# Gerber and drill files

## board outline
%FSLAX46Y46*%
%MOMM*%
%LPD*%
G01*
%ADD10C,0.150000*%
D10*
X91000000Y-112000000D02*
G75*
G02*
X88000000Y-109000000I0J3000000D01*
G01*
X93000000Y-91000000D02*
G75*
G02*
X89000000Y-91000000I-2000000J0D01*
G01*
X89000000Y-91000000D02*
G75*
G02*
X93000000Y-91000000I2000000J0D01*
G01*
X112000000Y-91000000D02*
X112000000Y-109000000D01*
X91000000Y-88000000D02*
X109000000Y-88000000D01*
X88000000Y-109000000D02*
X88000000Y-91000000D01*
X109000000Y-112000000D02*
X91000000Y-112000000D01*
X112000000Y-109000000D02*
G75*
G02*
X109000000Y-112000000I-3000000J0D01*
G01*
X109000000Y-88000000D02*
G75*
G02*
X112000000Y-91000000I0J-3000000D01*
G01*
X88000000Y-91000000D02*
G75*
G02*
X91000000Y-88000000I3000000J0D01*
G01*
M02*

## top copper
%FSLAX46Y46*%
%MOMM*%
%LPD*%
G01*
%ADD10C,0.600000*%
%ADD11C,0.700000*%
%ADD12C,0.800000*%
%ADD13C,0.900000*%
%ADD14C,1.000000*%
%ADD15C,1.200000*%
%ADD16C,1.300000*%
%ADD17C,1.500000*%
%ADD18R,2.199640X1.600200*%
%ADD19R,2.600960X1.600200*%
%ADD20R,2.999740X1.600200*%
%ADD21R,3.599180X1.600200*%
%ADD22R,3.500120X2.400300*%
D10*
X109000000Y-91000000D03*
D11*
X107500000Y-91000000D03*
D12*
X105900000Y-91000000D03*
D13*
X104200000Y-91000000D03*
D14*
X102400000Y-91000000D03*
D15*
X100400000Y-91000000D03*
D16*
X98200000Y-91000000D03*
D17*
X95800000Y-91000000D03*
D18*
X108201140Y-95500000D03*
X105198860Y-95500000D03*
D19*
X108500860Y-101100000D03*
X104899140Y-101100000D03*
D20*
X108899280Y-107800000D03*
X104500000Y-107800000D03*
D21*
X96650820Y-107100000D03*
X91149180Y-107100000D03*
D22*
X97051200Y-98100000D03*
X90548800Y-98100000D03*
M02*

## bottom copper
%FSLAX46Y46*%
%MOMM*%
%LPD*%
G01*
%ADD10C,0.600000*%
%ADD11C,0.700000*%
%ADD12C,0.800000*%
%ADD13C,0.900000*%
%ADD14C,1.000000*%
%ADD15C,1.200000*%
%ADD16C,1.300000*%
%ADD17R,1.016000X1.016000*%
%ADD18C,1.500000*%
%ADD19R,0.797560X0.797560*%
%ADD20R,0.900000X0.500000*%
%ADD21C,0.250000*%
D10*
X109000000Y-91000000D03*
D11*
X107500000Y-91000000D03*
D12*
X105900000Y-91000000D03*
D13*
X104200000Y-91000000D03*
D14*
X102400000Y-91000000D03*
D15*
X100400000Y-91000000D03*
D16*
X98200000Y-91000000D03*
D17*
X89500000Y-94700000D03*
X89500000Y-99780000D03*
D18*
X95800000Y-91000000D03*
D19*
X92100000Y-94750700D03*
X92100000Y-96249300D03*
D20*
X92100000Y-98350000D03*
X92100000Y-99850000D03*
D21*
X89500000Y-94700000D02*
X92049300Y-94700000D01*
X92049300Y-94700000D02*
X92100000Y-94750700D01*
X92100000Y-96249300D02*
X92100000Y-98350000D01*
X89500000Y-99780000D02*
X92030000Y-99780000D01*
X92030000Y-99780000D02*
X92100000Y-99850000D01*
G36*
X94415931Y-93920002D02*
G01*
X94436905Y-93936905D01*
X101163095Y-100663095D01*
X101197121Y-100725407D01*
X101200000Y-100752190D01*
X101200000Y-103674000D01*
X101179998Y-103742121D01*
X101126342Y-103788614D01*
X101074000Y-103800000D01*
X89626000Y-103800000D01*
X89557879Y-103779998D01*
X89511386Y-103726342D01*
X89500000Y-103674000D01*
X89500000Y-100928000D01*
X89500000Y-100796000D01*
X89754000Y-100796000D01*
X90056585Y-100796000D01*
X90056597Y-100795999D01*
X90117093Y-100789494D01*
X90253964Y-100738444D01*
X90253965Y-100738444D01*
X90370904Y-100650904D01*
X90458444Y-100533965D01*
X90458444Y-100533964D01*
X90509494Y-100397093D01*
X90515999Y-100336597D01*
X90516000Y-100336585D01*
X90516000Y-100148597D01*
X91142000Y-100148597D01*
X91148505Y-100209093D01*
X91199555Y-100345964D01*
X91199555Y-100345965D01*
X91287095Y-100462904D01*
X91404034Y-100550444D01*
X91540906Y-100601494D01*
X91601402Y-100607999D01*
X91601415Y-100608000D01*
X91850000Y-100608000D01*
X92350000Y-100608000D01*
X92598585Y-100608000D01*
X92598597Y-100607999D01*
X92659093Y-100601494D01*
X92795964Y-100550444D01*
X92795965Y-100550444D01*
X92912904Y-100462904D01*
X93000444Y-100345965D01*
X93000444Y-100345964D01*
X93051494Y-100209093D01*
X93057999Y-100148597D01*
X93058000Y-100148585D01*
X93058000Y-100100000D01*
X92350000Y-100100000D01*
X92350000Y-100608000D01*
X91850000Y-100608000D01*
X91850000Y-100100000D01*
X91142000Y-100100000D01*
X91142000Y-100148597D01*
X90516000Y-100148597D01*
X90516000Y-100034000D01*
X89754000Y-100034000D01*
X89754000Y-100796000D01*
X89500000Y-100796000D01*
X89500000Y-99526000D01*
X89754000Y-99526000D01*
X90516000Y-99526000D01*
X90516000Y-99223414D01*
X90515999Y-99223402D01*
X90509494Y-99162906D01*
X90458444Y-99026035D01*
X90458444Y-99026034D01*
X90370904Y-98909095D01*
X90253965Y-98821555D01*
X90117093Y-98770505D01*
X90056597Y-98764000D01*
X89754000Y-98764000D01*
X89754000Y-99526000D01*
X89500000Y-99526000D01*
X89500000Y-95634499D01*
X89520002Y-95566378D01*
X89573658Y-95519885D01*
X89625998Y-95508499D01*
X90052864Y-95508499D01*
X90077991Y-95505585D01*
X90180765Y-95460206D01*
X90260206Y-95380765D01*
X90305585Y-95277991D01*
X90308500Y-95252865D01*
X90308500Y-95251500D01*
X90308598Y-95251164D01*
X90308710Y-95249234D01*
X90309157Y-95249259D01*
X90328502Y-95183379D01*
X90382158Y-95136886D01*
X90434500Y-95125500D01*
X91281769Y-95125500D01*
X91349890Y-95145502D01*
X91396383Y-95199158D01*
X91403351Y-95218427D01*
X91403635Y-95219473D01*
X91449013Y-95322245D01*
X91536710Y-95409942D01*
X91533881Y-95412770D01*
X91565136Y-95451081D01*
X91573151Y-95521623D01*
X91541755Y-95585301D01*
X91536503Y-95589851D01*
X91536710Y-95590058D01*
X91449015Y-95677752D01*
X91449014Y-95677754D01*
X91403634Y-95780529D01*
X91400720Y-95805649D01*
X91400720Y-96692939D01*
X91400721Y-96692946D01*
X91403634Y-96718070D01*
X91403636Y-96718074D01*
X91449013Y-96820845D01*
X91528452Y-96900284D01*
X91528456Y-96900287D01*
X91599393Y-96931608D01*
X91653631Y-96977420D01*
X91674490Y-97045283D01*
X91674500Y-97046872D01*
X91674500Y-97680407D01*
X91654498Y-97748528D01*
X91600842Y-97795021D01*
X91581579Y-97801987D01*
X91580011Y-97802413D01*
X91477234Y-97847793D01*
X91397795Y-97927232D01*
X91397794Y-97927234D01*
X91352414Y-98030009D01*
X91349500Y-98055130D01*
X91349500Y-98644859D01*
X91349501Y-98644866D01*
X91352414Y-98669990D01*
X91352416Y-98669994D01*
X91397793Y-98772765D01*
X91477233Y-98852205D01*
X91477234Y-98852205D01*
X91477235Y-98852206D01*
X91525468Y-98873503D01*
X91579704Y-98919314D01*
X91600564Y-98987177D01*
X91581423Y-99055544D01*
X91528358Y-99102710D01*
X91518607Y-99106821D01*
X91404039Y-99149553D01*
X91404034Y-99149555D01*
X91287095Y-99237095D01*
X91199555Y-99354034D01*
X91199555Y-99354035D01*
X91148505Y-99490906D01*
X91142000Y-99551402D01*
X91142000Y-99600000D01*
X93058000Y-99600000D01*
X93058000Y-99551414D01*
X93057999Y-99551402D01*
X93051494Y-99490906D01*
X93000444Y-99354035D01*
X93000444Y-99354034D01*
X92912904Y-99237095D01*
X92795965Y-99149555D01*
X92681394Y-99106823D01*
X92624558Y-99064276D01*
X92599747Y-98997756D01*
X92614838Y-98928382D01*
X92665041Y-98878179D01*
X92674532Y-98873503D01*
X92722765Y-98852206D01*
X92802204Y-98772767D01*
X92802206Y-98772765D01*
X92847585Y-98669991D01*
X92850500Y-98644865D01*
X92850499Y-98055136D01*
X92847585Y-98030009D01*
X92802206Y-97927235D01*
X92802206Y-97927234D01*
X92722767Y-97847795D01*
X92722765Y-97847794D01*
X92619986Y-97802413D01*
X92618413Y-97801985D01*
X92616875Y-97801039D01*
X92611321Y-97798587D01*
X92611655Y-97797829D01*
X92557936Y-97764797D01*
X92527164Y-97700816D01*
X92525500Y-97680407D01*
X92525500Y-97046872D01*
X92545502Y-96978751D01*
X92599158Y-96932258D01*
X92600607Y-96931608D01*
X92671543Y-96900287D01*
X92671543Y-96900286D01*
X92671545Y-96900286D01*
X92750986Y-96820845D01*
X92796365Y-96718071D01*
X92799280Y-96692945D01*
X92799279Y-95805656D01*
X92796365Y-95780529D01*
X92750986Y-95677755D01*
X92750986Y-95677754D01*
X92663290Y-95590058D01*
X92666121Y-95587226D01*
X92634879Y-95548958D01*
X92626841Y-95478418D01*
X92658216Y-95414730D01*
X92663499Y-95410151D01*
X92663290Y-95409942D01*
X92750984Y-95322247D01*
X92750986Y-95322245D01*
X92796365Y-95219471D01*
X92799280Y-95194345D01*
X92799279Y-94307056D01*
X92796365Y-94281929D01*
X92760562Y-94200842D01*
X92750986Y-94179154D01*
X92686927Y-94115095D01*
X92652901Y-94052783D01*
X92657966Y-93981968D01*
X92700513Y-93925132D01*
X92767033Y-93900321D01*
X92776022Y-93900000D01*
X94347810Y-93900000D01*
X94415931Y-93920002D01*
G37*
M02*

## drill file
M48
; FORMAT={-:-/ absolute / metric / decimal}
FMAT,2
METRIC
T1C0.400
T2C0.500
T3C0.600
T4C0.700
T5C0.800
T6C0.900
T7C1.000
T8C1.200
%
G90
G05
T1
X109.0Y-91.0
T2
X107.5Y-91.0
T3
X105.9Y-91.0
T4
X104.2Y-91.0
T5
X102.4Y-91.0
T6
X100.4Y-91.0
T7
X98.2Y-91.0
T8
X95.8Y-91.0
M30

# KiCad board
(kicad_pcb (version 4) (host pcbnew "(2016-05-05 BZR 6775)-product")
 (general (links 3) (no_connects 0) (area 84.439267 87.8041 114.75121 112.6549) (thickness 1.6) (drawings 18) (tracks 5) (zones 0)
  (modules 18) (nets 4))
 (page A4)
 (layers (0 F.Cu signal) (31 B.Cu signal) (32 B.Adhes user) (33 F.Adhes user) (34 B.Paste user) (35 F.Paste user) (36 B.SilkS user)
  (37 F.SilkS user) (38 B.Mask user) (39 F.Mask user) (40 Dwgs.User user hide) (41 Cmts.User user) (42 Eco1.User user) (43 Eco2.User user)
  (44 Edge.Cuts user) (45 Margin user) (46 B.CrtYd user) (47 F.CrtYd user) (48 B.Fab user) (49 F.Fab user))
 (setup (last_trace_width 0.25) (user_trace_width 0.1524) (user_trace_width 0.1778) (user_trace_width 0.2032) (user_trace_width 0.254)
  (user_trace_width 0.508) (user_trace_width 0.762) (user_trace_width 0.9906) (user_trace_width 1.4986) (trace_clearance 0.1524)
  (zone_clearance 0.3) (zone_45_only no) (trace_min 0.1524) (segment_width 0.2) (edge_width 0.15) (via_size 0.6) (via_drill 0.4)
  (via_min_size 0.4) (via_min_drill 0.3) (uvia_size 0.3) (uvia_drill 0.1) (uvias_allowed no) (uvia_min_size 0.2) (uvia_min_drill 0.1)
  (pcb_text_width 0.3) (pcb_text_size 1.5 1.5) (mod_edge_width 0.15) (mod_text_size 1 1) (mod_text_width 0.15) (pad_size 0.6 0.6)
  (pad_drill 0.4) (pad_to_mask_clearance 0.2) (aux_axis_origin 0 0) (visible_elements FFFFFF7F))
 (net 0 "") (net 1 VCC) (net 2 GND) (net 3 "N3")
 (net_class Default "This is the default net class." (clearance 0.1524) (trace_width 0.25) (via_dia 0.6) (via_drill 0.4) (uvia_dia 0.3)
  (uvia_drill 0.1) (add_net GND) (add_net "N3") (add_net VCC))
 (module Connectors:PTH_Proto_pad (layer F.Cu) (at 109 91)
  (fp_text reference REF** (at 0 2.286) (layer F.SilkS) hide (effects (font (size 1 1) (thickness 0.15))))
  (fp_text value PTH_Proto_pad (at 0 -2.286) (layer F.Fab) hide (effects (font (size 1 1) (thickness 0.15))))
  (pad 1 thru_hole circle (at 0 0) (size 0.6 0.6) (drill 0.4) (layers *.Cu *.Mask F.SilkS)))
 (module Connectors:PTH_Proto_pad (layer F.Cu) (at 107.5 91)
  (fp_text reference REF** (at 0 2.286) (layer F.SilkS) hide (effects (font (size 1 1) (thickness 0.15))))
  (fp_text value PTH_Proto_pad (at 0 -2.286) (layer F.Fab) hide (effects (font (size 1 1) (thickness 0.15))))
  (pad 1 thru_hole circle (at 0 0) (size 0.7 0.7) (drill 0.5) (layers *.Cu *.Mask F.SilkS)))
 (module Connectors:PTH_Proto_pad (layer F.Cu) (at 105.9 91)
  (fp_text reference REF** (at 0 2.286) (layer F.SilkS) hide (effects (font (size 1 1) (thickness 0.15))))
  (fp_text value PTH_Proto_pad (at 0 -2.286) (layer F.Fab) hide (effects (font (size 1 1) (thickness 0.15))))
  (pad 1 thru_hole circle (at 0 0) (size 0.8 0.8) (drill 0.6) (layers *.Cu *.Mask F.SilkS)))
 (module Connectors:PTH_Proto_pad (layer F.Cu) (at 104.2 91)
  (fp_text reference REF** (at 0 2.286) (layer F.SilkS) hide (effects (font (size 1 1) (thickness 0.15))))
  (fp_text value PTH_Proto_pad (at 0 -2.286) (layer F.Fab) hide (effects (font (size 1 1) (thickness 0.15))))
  (pad 1 thru_hole circle (at 0 0) (size 0.9 0.9) (drill 0.7) (layers *.Cu *.Mask F.SilkS)))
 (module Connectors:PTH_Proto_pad (layer F.Cu) (at 102.4 91)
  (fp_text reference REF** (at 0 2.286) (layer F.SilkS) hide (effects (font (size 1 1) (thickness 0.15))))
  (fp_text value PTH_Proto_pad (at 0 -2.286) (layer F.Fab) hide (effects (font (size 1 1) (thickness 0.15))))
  (pad 1 thru_hole circle (at 0 0) (size 1 1) (drill 0.8) (layers *.Cu *.Mask F.SilkS)))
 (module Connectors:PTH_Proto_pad (layer F.Cu) (at 100.4 91)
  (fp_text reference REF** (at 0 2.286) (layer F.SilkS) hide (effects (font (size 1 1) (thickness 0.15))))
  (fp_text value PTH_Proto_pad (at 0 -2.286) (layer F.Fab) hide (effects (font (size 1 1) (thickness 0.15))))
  (pad 1 thru_hole circle (at 0 0) (size 1.2 1.2) (drill 0.9) (layers *.Cu *.Mask F.SilkS)))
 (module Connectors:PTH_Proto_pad (layer F.Cu) (at 98.2 91)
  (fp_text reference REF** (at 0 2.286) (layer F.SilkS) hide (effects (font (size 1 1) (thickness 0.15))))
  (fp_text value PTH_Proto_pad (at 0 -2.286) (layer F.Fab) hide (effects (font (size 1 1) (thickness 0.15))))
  (pad 1 thru_hole circle (at 0 0) (size 1.3 1.3) (drill 1) (layers *.Cu *.Mask F.SilkS)))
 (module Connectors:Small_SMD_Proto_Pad (layer B.Cu) (at 89.5 94.7)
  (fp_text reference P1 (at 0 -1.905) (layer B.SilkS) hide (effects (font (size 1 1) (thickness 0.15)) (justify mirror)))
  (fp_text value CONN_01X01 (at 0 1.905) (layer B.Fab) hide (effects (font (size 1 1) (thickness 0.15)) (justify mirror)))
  (pad 1 smd rect (at 0 0) (size 1.016 1.016) (layers B.Cu B.Paste B.Mask) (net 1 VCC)))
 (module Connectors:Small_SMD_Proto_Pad (layer B.Cu) (at 89.5 99.78)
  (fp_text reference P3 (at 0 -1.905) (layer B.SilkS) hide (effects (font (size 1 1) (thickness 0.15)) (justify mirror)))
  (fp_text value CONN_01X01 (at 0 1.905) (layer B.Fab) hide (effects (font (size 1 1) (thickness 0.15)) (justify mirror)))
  (pad 1 smd rect (at 0 0) (size 1.016 1.016) (layers B.Cu B.Paste B.Mask) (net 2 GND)))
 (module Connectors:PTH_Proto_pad (layer F.Cu) (at 95.8 91)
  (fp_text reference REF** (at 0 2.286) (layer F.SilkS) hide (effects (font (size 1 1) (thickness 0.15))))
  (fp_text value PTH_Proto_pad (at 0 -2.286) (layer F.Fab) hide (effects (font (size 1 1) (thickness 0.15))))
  (pad 1 thru_hole circle (at 0 0) (size 1.5 1.5) (drill 1.2) (layers *.Cu *.Mask F.SilkS)))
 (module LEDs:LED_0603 (layer B.Cu) (at 92.1 95.5 90)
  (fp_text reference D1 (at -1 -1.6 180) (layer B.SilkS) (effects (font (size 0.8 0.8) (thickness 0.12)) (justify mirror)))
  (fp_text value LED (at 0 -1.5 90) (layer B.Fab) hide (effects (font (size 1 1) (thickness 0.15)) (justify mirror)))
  (pad 2 smd rect (at 0.7493 0 270) (size 0.79756 0.79756) (layers B.Cu B.Paste B.Mask) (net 1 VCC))
  (pad 1 smd rect (at -0.7493 0 270) (size 0.79756 0.79756) (layers B.Cu B.Paste B.Mask) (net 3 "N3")))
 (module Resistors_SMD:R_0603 (layer B.Cu) (at 92.1 99.1 270)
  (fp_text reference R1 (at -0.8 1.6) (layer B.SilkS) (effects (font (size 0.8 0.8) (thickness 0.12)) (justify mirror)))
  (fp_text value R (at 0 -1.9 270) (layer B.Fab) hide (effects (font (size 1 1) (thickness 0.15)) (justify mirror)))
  (pad 1 smd rect (at -0.75 0 270) (size 0.5 0.9) (layers B.Cu B.Paste B.Mask) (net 3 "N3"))
  (pad 2 smd rect (at 0.75 0 270) (size 0.5 0.9) (layers B.Cu B.Paste B.Mask) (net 2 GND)))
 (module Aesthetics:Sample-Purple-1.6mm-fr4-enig (layer B.Cu) (at 100 102.6 180)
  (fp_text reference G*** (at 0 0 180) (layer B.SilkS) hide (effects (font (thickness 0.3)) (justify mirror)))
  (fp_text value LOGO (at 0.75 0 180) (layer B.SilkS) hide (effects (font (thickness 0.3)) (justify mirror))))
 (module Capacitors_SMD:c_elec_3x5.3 (layer F.Cu) (at 106.7 95.5)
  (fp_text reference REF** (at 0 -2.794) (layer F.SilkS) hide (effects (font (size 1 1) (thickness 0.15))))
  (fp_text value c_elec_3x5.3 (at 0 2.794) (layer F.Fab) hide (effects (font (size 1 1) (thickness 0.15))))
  (pad 1 smd rect (at 1.50114 0) (size 2.19964 1.6002) (layers F.Cu F.Paste F.Mask))
  (pad 2 smd rect (at -1.50114 0) (size 2.19964 1.6002) (layers F.Cu F.Paste F.Mask)))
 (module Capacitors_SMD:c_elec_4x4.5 (layer F.Cu) (at 106.7 101.1)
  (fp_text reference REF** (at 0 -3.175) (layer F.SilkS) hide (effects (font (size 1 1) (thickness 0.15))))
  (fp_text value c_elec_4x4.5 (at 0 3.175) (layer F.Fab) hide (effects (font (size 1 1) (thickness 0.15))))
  (pad 1 smd rect (at 1.80086 0) (size 2.60096 1.6002) (layers F.Cu F.Paste F.Mask))
  (pad 2 smd rect (at -1.80086 0) (size 2.60096 1.6002) (layers F.Cu F.Paste F.Mask)))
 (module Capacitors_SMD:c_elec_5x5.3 (layer F.Cu) (at 106.69964 107.8)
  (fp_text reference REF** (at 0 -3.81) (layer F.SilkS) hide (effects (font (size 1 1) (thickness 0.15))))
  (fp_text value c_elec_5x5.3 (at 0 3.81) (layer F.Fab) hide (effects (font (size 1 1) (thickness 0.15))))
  (pad 1 smd rect (at 2.19964 0) (size 2.99974 1.6002) (layers F.Cu F.Paste F.Mask))
  (pad 2 smd rect (at -2.19964 0) (size 2.99974 1.6002) (layers F.Cu F.Paste F.Mask)))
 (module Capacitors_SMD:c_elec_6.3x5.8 (layer F.Cu) (at 93.9 107.1)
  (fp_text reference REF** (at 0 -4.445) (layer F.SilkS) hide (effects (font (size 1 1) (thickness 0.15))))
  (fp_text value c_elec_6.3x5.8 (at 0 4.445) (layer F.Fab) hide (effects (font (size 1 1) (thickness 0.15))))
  (pad 1 smd rect (at 2.75082 0) (size 3.59918 1.6002) (layers F.Cu F.Paste F.Mask))
  (pad 2 smd rect (at -2.75082 0) (size 3.59918 1.6002) (layers F.Cu F.Paste F.Mask)))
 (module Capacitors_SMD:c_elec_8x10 (layer F.Cu) (at 93.8 98.1)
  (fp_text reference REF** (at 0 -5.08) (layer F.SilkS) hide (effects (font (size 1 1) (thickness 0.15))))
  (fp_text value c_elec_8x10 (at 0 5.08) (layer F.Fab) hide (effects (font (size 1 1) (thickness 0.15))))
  (pad 1 smd rect (at 3.2512 0) (size 3.50012 2.4003) (layers F.Cu F.Paste F.Mask))
  (pad 2 smd rect (at -3.2512 0) (size 3.50012 2.4003) (layers F.Cu F.Paste F.Mask)))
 (gr_arc (start 91 109) (end 91 112) (angle 90) (layer Edge.Cuts) (width 0.15))
 (gr_circle (center 91 91) (end 93 91) (layer Edge.Cuts) (width 0.15))
 (gr_line (start 112 91) (end 112 109) (layer Edge.Cuts) (width 0.15))
 (gr_line (start 91 88) (end 109 88) (layer Edge.Cuts) (width 0.15))
 (gr_line (start 88 109) (end 88 91) (layer Edge.Cuts) (width 0.15))
 (gr_line (start 109 112) (end 91 112) (layer Edge.Cuts) (width 0.15))
 (gr_arc (start 109 109) (end 112 109) (angle 90) (layer Edge.Cuts) (width 0.15))
 (gr_arc (start 109 91) (end 109 88) (angle 90) (layer Edge.Cuts) (width 0.15))
 (gr_arc (start 91 91) (end 88 91) (angle 90) (layer Edge.Cuts) (width 0.15))
 (segment (start 89.5 94.7) (end 92.0493 94.7) (width 0.25) (layer B.Cu) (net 1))
 (segment (start 92.0493 94.7) (end 92.1 94.7507) (width 0.25) (layer B.Cu) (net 1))
 (segment (start 92.1 96.2493) (end 92.1 98.35) (width 0.25) (layer B.Cu) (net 3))
 (segment (start 89.5 99.78) (end 92.03 99.78) (width 0.25) (layer B.Cu) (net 2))
 (segment (start 92.03 99.78) (end 92.1 99.85) (width 0.25) (layer B.Cu) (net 2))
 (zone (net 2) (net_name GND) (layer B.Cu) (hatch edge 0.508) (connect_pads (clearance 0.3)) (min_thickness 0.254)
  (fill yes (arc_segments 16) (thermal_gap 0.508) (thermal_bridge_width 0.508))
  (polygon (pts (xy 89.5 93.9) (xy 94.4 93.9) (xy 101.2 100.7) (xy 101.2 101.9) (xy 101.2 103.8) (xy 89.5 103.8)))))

